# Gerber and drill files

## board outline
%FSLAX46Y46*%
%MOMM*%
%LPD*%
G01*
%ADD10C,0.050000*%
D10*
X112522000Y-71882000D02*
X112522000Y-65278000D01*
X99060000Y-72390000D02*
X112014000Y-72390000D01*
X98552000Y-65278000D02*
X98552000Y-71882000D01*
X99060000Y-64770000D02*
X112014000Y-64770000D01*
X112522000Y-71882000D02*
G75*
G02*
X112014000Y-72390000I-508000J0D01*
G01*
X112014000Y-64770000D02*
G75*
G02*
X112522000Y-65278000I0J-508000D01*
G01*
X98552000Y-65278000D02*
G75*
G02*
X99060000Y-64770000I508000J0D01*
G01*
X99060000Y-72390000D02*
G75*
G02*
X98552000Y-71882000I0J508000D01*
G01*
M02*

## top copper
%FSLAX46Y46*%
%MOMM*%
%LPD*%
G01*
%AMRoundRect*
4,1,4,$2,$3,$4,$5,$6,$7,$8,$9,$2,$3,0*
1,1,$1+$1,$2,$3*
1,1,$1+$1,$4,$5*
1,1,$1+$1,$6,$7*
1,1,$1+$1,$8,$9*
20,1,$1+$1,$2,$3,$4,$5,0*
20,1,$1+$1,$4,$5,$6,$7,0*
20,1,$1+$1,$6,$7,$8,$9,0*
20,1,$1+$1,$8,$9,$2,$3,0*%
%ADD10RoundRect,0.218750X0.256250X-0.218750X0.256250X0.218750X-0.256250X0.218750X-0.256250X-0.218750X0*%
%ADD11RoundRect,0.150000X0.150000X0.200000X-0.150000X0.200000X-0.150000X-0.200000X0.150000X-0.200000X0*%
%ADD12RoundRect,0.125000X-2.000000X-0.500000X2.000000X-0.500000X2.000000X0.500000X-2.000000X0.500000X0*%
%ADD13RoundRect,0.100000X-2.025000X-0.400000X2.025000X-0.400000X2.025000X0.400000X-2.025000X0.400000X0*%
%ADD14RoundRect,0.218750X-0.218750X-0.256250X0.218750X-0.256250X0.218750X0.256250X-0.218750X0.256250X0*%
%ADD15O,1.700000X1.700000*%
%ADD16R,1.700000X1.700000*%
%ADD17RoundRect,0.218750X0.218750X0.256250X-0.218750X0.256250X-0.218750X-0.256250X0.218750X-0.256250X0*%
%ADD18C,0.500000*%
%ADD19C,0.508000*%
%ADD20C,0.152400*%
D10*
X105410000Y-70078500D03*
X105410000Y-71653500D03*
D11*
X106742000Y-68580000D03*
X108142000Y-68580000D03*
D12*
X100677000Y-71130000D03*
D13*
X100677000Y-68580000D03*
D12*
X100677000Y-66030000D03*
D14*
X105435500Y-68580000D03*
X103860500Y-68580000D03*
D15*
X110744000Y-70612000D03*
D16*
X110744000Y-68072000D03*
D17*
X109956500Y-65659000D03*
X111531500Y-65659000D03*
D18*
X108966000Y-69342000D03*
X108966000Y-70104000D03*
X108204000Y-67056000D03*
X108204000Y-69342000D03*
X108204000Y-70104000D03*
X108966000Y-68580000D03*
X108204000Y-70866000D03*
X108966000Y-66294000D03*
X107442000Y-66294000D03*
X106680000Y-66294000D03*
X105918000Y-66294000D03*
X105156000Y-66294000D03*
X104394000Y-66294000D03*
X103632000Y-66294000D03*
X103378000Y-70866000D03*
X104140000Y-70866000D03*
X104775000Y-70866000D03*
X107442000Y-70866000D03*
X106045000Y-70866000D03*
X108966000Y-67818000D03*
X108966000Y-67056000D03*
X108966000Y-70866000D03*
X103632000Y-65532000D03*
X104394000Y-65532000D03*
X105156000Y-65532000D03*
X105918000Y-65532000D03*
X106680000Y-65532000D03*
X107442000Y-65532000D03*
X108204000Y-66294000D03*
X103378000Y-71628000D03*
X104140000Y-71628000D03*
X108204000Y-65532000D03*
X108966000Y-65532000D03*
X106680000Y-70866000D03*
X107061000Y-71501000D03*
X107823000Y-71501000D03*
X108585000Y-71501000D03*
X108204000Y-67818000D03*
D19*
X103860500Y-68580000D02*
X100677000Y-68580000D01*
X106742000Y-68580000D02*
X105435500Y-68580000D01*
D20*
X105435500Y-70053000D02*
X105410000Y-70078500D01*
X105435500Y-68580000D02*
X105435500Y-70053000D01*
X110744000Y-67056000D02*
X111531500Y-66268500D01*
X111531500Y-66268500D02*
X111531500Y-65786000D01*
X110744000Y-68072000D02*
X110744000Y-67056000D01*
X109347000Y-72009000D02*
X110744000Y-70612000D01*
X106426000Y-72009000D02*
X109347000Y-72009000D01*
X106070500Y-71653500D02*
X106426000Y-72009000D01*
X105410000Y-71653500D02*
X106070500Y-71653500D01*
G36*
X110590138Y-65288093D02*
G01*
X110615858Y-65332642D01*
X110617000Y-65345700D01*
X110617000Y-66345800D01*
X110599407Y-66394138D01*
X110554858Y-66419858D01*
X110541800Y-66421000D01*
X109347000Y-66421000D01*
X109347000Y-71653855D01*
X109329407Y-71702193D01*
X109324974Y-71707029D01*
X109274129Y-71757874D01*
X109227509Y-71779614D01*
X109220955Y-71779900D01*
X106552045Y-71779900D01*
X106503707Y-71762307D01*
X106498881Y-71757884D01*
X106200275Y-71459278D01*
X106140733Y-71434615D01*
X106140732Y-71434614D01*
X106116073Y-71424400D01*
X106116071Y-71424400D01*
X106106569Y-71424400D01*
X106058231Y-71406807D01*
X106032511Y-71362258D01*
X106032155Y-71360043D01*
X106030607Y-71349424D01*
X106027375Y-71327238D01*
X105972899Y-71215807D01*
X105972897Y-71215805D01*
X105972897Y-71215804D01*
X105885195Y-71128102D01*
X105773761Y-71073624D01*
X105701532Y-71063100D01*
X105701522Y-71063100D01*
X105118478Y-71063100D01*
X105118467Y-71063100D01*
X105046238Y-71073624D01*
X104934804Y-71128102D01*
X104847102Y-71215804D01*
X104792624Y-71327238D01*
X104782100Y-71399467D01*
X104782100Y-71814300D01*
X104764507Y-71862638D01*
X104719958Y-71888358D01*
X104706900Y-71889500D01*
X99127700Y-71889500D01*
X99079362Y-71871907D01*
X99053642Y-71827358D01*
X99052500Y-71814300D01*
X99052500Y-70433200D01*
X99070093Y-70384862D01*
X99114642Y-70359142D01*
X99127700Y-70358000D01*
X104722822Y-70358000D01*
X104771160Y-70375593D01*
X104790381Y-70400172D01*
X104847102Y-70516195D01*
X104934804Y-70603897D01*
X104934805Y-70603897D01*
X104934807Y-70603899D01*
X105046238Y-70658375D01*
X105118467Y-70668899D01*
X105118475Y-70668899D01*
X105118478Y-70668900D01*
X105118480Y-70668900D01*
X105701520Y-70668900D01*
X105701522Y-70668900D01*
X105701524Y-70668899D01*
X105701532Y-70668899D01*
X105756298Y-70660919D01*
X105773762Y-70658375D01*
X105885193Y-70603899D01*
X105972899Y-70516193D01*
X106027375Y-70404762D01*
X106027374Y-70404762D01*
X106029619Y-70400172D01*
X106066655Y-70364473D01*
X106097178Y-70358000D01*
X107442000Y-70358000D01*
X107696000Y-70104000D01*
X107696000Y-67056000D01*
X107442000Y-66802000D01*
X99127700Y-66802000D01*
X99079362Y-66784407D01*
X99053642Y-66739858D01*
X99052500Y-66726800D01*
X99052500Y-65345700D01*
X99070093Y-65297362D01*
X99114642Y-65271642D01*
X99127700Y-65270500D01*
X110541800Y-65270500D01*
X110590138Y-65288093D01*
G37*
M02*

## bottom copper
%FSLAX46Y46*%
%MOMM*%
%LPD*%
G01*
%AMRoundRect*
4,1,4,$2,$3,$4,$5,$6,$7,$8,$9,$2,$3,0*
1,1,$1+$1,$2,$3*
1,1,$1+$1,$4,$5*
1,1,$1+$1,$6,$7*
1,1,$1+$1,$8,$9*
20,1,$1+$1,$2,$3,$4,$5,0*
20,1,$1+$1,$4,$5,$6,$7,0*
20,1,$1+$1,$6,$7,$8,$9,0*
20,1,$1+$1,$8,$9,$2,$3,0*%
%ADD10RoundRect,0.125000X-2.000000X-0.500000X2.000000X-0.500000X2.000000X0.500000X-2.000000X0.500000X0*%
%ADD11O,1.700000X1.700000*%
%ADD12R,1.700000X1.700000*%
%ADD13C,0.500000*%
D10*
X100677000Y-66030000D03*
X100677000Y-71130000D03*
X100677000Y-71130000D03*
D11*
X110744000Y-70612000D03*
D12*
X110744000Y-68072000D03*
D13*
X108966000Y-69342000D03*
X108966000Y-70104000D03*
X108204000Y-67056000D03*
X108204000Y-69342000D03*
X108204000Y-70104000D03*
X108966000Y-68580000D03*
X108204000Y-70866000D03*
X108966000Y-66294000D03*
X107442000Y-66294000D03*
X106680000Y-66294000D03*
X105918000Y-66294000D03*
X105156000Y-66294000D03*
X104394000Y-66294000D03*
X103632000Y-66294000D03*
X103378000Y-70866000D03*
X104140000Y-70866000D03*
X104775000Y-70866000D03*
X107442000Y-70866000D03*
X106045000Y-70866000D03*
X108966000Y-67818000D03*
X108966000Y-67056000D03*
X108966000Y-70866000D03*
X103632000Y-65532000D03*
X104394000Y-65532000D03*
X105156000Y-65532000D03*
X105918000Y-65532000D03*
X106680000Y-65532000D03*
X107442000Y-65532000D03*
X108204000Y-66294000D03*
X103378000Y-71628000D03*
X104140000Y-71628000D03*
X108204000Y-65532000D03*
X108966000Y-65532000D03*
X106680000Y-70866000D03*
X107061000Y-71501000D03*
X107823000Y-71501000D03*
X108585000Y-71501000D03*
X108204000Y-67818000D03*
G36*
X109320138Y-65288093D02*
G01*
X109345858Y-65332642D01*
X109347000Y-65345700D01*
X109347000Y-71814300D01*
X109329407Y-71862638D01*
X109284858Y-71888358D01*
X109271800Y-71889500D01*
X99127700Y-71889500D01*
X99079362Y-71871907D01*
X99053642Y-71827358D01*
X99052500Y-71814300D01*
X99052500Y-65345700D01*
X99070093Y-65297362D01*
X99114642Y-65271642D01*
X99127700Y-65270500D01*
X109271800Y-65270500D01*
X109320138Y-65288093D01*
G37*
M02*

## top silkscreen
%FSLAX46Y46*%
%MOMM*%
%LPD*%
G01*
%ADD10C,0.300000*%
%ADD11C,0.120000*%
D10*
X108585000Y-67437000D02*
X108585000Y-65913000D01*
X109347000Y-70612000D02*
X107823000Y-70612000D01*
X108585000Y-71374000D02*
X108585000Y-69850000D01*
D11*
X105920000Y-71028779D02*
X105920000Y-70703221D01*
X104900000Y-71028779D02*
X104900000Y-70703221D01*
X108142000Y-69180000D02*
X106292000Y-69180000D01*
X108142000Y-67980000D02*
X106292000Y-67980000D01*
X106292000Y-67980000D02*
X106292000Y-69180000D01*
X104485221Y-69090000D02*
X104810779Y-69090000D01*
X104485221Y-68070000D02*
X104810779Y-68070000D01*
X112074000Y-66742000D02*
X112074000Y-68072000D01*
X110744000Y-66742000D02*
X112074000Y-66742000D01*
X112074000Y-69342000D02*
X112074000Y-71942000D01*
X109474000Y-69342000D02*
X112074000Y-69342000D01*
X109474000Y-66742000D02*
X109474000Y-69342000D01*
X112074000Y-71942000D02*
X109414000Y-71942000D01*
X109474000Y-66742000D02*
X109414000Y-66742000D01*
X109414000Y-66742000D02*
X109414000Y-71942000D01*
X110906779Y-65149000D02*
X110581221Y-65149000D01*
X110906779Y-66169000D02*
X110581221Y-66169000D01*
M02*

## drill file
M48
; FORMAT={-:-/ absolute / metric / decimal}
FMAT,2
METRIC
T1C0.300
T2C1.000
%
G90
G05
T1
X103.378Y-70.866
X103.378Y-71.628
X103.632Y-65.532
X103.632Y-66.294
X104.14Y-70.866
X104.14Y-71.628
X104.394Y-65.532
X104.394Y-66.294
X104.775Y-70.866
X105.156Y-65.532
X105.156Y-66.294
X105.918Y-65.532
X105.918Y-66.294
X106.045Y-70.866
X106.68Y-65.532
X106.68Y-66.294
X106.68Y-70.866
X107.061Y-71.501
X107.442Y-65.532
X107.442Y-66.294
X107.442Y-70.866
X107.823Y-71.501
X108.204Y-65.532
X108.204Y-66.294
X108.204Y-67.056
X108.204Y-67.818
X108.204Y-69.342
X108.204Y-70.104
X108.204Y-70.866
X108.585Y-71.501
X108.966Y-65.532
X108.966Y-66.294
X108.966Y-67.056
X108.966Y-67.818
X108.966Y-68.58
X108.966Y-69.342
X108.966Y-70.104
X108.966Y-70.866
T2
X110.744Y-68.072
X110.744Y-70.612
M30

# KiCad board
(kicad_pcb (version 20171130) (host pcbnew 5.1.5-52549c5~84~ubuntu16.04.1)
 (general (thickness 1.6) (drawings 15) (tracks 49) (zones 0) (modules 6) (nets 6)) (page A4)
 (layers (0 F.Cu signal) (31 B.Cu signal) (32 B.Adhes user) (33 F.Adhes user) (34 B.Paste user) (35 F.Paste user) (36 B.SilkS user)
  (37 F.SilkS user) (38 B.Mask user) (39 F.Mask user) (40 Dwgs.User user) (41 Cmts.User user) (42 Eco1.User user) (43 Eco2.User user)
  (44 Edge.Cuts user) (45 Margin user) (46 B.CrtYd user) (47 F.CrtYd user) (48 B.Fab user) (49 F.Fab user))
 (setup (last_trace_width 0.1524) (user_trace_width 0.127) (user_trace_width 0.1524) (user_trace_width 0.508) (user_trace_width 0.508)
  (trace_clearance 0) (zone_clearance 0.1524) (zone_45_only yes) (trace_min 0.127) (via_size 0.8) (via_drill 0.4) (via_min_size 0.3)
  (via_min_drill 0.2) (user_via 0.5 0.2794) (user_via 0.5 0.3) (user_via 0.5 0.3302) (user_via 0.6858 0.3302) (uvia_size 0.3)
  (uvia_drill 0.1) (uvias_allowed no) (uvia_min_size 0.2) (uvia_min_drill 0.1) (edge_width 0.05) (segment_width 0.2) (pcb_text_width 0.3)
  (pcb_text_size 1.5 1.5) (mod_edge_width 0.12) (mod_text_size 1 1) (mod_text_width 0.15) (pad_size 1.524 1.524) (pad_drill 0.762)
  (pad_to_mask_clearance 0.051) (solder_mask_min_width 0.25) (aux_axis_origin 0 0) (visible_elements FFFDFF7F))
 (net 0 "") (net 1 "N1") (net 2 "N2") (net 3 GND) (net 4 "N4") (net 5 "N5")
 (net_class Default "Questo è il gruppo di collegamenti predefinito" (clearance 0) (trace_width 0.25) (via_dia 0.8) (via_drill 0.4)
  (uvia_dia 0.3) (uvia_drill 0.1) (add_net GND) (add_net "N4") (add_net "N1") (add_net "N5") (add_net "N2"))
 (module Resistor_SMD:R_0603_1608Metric (layer F.Cu) (at 105.41 70.866 90)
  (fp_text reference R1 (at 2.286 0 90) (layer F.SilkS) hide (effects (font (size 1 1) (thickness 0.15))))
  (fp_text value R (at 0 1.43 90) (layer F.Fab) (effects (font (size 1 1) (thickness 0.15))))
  (fp_line (start -0.162779 0.51) (end 0.162779 0.51) (layer F.SilkS) (width 0.12))
  (fp_line (start -0.162779 -0.51) (end 0.162779 -0.51) (layer F.SilkS) (width 0.12))
  (pad 2 smd roundrect (at 0.7875 0 90) (size 0.875 0.95) (layers F.Cu F.Paste F.Mask) (roundrect_rratio 0.25) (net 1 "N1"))
  (pad 1 smd roundrect (at -0.7875 0 90) (size 0.875 0.95) (layers F.Cu F.Paste F.Mask) (roundrect_rratio 0.25) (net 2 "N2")))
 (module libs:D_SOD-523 (layer F.Cu) (at 107.442 68.58)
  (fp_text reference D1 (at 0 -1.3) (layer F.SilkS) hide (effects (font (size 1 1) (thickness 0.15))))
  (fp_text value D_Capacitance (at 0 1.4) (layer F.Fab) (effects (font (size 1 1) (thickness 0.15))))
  (fp_line (start 0.7 0.6) (end -1.15 0.6) (layer F.SilkS) (width 0.12))
  (fp_line (start 0.7 -0.6) (end -1.15 -0.6) (layer F.SilkS) (width 0.12))
  (fp_line (start -1.15 -0.6) (end -1.15 0.6) (layer F.SilkS) (width 0.12))
  (pad 1 smd roundrect (at -0.7 0 180) (size 0.6 0.7) (layers F.Cu F.Paste F.Mask) (roundrect_rratio 0.25) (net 1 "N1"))
  (pad 2 smd roundrect (at 0.7 0 180) (size 0.6 0.7) (layers F.Cu F.Paste F.Mask) (roundrect_rratio 0.25) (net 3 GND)))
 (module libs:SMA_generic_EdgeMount (layer F.Cu) (at 98.552 68.58)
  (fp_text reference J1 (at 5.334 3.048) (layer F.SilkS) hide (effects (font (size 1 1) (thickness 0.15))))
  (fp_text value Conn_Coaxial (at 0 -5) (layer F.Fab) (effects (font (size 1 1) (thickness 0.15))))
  (pad 2 smd roundrect (at 2.125 -2.55) (size 4.25 1.25) (layers B.Cu B.Paste B.Mask) (roundrect_rratio 0.1) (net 3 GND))
  (pad 2 smd roundrect (at 2.125 2.55) (size 4.25 1.25) (layers F.Cu F.Paste F.Mask) (roundrect_rratio 0.1) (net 3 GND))
  (pad 2 smd roundrect (at 2.125 2.55) (size 4.25 1.25) (layers B.Cu B.Paste B.Mask) (roundrect_rratio 0.1) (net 3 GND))
  (pad 1 smd roundrect (at 2.125 0) (size 4.25 1) (layers F.Cu F.Paste F.Mask) (roundrect_rratio 0.1) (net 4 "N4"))
  (pad 2 smd roundrect (at 2.125 -2.55) (size 4.25 1.25) (layers F.Cu F.Paste F.Mask) (roundrect_rratio 0.1) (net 3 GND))
  (pad 2 smd roundrect (at 2.125 2.55) (size 4.25 1.25) (layers B.Cu B.Paste B.Mask) (roundrect_rratio 0.1) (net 3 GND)))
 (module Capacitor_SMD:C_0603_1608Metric (layer F.Cu) (at 104.648 68.58)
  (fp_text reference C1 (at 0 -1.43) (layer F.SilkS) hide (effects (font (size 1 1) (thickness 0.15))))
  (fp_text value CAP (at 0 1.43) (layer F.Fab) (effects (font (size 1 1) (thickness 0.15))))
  (fp_line (start -0.162779 0.51) (end 0.162779 0.51) (layer F.SilkS) (width 0.12))
  (fp_line (start -0.162779 -0.51) (end 0.162779 -0.51) (layer F.SilkS) (width 0.12))
  (pad 2 smd roundrect (at 0.7875 0) (size 0.875 0.95) (layers F.Cu F.Paste F.Mask) (roundrect_rratio 0.25) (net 1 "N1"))
  (pad 1 smd roundrect (at -0.7875 0) (size 0.875 0.95) (layers F.Cu F.Paste F.Mask) (roundrect_rratio 0.25) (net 4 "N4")))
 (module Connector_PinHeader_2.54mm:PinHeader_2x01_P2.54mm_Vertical (layer F.Cu) (at 110.744 68.072 270)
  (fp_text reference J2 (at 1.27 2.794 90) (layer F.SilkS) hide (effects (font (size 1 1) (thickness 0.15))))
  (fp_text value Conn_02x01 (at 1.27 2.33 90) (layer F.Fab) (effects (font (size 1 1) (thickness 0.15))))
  (fp_line (start -1.33 -1.33) (end 0 -1.33) (layer F.SilkS) (width 0.12))
  (fp_line (start -1.33 0) (end -1.33 -1.33) (layer F.SilkS) (width 0.12))
  (fp_line (start 1.27 -1.33) (end 3.87 -1.33) (layer F.SilkS) (width 0.12))
  (fp_line (start 1.27 1.27) (end 1.27 -1.33) (layer F.SilkS) (width 0.12))
  (fp_line (start -1.33 1.27) (end 1.27 1.27) (layer F.SilkS) (width 0.12))
  (fp_line (start 3.87 -1.33) (end 3.87 1.33) (layer F.SilkS) (width 0.12))
  (fp_line (start -1.33 1.27) (end -1.33 1.33) (layer F.SilkS) (width 0.12))
  (fp_line (start -1.33 1.33) (end 3.87 1.33) (layer F.SilkS) (width 0.12))
  (pad 2 thru_hole oval (at 2.54 0 270) (size 1.7 1.7) (drill 1) (layers *.Cu *.Mask) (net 2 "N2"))
  (pad 1 thru_hole rect (at 0 0 270) (size 1.7 1.7) (drill 1) (layers *.Cu *.Mask) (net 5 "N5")))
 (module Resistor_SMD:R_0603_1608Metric (layer F.Cu) (at 110.744 65.659 180)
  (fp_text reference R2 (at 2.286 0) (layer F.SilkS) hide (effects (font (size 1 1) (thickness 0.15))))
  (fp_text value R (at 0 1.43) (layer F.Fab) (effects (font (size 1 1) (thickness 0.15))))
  (fp_line (start -0.162779 0.51) (end 0.162779 0.51) (layer F.SilkS) (width 0.12))
  (fp_line (start -0.162779 -0.51) (end 0.162779 -0.51) (layer F.SilkS) (width 0.12))
  (pad 2 smd roundrect (at 0.7875 0 180) (size 0.875 0.95) (layers F.Cu F.Paste F.Mask) (roundrect_rratio 0.25) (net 3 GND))
  (pad 1 smd roundrect (at -0.7875 0 180) (size 0.875 0.95) (layers F.Cu F.Paste F.Mask) (roundrect_rratio 0.25) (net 5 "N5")))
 (gr_line (start 108.585 67.437) (end 108.585 65.913) (layer F.SilkS) (width 0.3))
 (gr_line (start 109.347 70.612) (end 107.823 70.612) (layer F.SilkS) (width 0.3))
 (gr_line (start 108.585 71.374) (end 108.585 69.85) (layer F.SilkS) (width 0.3))
 (gr_line (start 112.522 71.882) (end 112.522 65.278) (layer Edge.Cuts) (width 0.05))
 (gr_line (start 99.06 72.39) (end 112.014 72.39) (layer Edge.Cuts) (width 0.05))
 (gr_line (start 98.552 65.278) (end 98.552 71.882) (layer Edge.Cuts) (width 0.05))
 (gr_line (start 99.06 64.77) (end 112.014 64.77) (layer Edge.Cuts) (width 0.05))
 (gr_arc (start 112.014 71.882) (end 112.014 72.39) (angle -90) (layer Edge.Cuts) (width 0.05))
 (gr_arc (start 112.014 65.278) (end 112.522 65.278) (angle -90) (layer Edge.Cuts) (width 0.05))
 (gr_arc (start 99.06 65.278) (end 99.06 64.77) (angle -90) (layer Edge.Cuts) (width 0.05))
 (gr_arc (start 99.06 71.882) (end 98.552 71.882) (angle -90) (layer Edge.Cuts) (width 0.05))
 (segment (start 103.8605 68.58) (end 100.677 68.58) (width 0.508) (layer F.Cu) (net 4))
 (segment (start 106.742 68.58) (end 105.4355 68.58) (width 0.508) (layer F.Cu) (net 1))
 (segment (start 105.4355 70.053) (end 105.41 70.0785) (width 0.1524) (layer F.Cu) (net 1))
 (segment (start 105.4355 68.58) (end 105.4355 70.053) (width 0.1524) (layer F.Cu) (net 1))
 (via (at 108.966 69.342) (size 0.5) (drill 0.3) (layers F.Cu B.Cu) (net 3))
 (via (at 108.966 70.104) (size 0.5) (drill 0.3) (layers F.Cu B.Cu) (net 3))
 (via (at 108.204 67.056) (size 0.5) (drill 0.3) (layers F.Cu B.Cu) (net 3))
 (via (at 108.204 69.342) (size 0.5) (drill 0.3) (layers F.Cu B.Cu) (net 3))
 (via (at 108.204 70.104) (size 0.5) (drill 0.3) (layers F.Cu B.Cu) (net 3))
 (via (at 108.966 68.58) (size 0.5) (drill 0.3) (layers F.Cu B.Cu) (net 3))
 (via (at 108.204 70.866) (size 0.5) (drill 0.3) (layers F.Cu B.Cu) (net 3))
 (via (at 108.966 66.294) (size 0.5) (drill 0.3) (layers F.Cu B.Cu) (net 3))
 (via (at 107.442 66.294) (size 0.5) (drill 0.3) (layers F.Cu B.Cu) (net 3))
 (via (at 106.68 66.294) (size 0.5) (drill 0.3) (layers F.Cu B.Cu) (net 3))
 (via (at 105.918 66.294) (size 0.5) (drill 0.3) (layers F.Cu B.Cu) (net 3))
 (via (at 105.156 66.294) (size 0.5) (drill 0.3) (layers F.Cu B.Cu) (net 3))
 (via (at 104.394 66.294) (size 0.5) (drill 0.3) (layers F.Cu B.Cu) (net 3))
 (via (at 103.632 66.294) (size 0.5) (drill 0.3) (layers F.Cu B.Cu) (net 3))
 (via (at 103.378 70.866) (size 0.5) (drill 0.3) (layers F.Cu B.Cu) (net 3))
 (via (at 104.14 70.866) (size 0.5) (drill 0.3) (layers F.Cu B.Cu) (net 3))
 (via (at 104.775 70.866) (size 0.5) (drill 0.3) (layers F.Cu B.Cu) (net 3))
 (via (at 107.442 70.866) (size 0.5) (drill 0.3) (layers F.Cu B.Cu) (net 3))
 (via (at 106.045 70.866) (size 0.5) (drill 0.3) (layers F.Cu B.Cu) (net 3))
 (via (at 108.966 67.818) (size 0.5) (drill 0.3) (layers F.Cu B.Cu) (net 3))
 (via (at 108.966 67.056) (size 0.5) (drill 0.3) (layers F.Cu B.Cu) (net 3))
 (via (at 108.966 70.866) (size 0.5) (drill 0.3) (layers F.Cu B.Cu) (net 3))
 (via (at 103.632 65.532) (size 0.5) (drill 0.3) (layers F.Cu B.Cu) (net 3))
 (via (at 104.394 65.532) (size 0.5) (drill 0.3) (layers F.Cu B.Cu) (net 3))
 (via (at 105.156 65.532) (size 0.5) (drill 0.3) (layers F.Cu B.Cu) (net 3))
 (via (at 105.918 65.532) (size 0.5) (drill 0.3) (layers F.Cu B.Cu) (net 3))
 (via (at 106.68 65.532) (size 0.5) (drill 0.3) (layers F.Cu B.Cu) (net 3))
 (via (at 107.442 65.532) (size 0.5) (drill 0.3) (layers F.Cu B.Cu) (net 3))
 (via (at 108.204 66.294) (size 0.5) (drill 0.3) (layers F.Cu B.Cu) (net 3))
 (via (at 103.378 71.628) (size 0.5) (drill 0.3) (layers F.Cu B.Cu) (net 3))
 (via (at 104.14 71.628) (size 0.5) (drill 0.3) (layers F.Cu B.Cu) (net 3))
 (via (at 108.204 65.532) (size 0.5) (drill 0.3) (layers F.Cu B.Cu) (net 3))
 (via (at 108.966 65.532) (size 0.5) (drill 0.3) (layers F.Cu B.Cu) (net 3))
 (via (at 106.68 70.866) (size 0.5) (drill 0.3) (layers F.Cu B.Cu) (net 3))
 (via (at 107.061 71.501) (size 0.5) (drill 0.3) (layers F.Cu B.Cu) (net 3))
 (via (at 107.823 71.501) (size 0.5) (drill 0.3) (layers F.Cu B.Cu) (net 3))
 (via (at 108.585 71.501) (size 0.5) (drill 0.3) (layers F.Cu B.Cu) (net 3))
 (via (at 108.204 67.818) (size 0.5) (drill 0.3) (layers F.Cu B.Cu) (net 3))
 (segment (start 110.744 67.056) (end 111.5315 66.2685) (width 0.1524) (layer F.Cu) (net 5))
 (segment (start 111.5315 66.2685) (end 111.5315 65.786) (width 0.1524) (layer F.Cu) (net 5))
 (segment (start 110.744 68.072) (end 110.744 67.056) (width 0.1524) (layer F.Cu) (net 5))
 (segment (start 109.347 72.009) (end 110.744 70.612) (width 0.1524) (layer F.Cu) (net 2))
 (segment (start 106.426 72.009) (end 109.347 72.009) (width 0.1524) (layer F.Cu) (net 2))
 (segment (start 106.0705 71.6535) (end 106.426 72.009) (width 0.1524) (layer F.Cu) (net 2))
 (segment (start 105.41 71.6535) (end 106.0705 71.6535) (width 0.1524) (layer F.Cu) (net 2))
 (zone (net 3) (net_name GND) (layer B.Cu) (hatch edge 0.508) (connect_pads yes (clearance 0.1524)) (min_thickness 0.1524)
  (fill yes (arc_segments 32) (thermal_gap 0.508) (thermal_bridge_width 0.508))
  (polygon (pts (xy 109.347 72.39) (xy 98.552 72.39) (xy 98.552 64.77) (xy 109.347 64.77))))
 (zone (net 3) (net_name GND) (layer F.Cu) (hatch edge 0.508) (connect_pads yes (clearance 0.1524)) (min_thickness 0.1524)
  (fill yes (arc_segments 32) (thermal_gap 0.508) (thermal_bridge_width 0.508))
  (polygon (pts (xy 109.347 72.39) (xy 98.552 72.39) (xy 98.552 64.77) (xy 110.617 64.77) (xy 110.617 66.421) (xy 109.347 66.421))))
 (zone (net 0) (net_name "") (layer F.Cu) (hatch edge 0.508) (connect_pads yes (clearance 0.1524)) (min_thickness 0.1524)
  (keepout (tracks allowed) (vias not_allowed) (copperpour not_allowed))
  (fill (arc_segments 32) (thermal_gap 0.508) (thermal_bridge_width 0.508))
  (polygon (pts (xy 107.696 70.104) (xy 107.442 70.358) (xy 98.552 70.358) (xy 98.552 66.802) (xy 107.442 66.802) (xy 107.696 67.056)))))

